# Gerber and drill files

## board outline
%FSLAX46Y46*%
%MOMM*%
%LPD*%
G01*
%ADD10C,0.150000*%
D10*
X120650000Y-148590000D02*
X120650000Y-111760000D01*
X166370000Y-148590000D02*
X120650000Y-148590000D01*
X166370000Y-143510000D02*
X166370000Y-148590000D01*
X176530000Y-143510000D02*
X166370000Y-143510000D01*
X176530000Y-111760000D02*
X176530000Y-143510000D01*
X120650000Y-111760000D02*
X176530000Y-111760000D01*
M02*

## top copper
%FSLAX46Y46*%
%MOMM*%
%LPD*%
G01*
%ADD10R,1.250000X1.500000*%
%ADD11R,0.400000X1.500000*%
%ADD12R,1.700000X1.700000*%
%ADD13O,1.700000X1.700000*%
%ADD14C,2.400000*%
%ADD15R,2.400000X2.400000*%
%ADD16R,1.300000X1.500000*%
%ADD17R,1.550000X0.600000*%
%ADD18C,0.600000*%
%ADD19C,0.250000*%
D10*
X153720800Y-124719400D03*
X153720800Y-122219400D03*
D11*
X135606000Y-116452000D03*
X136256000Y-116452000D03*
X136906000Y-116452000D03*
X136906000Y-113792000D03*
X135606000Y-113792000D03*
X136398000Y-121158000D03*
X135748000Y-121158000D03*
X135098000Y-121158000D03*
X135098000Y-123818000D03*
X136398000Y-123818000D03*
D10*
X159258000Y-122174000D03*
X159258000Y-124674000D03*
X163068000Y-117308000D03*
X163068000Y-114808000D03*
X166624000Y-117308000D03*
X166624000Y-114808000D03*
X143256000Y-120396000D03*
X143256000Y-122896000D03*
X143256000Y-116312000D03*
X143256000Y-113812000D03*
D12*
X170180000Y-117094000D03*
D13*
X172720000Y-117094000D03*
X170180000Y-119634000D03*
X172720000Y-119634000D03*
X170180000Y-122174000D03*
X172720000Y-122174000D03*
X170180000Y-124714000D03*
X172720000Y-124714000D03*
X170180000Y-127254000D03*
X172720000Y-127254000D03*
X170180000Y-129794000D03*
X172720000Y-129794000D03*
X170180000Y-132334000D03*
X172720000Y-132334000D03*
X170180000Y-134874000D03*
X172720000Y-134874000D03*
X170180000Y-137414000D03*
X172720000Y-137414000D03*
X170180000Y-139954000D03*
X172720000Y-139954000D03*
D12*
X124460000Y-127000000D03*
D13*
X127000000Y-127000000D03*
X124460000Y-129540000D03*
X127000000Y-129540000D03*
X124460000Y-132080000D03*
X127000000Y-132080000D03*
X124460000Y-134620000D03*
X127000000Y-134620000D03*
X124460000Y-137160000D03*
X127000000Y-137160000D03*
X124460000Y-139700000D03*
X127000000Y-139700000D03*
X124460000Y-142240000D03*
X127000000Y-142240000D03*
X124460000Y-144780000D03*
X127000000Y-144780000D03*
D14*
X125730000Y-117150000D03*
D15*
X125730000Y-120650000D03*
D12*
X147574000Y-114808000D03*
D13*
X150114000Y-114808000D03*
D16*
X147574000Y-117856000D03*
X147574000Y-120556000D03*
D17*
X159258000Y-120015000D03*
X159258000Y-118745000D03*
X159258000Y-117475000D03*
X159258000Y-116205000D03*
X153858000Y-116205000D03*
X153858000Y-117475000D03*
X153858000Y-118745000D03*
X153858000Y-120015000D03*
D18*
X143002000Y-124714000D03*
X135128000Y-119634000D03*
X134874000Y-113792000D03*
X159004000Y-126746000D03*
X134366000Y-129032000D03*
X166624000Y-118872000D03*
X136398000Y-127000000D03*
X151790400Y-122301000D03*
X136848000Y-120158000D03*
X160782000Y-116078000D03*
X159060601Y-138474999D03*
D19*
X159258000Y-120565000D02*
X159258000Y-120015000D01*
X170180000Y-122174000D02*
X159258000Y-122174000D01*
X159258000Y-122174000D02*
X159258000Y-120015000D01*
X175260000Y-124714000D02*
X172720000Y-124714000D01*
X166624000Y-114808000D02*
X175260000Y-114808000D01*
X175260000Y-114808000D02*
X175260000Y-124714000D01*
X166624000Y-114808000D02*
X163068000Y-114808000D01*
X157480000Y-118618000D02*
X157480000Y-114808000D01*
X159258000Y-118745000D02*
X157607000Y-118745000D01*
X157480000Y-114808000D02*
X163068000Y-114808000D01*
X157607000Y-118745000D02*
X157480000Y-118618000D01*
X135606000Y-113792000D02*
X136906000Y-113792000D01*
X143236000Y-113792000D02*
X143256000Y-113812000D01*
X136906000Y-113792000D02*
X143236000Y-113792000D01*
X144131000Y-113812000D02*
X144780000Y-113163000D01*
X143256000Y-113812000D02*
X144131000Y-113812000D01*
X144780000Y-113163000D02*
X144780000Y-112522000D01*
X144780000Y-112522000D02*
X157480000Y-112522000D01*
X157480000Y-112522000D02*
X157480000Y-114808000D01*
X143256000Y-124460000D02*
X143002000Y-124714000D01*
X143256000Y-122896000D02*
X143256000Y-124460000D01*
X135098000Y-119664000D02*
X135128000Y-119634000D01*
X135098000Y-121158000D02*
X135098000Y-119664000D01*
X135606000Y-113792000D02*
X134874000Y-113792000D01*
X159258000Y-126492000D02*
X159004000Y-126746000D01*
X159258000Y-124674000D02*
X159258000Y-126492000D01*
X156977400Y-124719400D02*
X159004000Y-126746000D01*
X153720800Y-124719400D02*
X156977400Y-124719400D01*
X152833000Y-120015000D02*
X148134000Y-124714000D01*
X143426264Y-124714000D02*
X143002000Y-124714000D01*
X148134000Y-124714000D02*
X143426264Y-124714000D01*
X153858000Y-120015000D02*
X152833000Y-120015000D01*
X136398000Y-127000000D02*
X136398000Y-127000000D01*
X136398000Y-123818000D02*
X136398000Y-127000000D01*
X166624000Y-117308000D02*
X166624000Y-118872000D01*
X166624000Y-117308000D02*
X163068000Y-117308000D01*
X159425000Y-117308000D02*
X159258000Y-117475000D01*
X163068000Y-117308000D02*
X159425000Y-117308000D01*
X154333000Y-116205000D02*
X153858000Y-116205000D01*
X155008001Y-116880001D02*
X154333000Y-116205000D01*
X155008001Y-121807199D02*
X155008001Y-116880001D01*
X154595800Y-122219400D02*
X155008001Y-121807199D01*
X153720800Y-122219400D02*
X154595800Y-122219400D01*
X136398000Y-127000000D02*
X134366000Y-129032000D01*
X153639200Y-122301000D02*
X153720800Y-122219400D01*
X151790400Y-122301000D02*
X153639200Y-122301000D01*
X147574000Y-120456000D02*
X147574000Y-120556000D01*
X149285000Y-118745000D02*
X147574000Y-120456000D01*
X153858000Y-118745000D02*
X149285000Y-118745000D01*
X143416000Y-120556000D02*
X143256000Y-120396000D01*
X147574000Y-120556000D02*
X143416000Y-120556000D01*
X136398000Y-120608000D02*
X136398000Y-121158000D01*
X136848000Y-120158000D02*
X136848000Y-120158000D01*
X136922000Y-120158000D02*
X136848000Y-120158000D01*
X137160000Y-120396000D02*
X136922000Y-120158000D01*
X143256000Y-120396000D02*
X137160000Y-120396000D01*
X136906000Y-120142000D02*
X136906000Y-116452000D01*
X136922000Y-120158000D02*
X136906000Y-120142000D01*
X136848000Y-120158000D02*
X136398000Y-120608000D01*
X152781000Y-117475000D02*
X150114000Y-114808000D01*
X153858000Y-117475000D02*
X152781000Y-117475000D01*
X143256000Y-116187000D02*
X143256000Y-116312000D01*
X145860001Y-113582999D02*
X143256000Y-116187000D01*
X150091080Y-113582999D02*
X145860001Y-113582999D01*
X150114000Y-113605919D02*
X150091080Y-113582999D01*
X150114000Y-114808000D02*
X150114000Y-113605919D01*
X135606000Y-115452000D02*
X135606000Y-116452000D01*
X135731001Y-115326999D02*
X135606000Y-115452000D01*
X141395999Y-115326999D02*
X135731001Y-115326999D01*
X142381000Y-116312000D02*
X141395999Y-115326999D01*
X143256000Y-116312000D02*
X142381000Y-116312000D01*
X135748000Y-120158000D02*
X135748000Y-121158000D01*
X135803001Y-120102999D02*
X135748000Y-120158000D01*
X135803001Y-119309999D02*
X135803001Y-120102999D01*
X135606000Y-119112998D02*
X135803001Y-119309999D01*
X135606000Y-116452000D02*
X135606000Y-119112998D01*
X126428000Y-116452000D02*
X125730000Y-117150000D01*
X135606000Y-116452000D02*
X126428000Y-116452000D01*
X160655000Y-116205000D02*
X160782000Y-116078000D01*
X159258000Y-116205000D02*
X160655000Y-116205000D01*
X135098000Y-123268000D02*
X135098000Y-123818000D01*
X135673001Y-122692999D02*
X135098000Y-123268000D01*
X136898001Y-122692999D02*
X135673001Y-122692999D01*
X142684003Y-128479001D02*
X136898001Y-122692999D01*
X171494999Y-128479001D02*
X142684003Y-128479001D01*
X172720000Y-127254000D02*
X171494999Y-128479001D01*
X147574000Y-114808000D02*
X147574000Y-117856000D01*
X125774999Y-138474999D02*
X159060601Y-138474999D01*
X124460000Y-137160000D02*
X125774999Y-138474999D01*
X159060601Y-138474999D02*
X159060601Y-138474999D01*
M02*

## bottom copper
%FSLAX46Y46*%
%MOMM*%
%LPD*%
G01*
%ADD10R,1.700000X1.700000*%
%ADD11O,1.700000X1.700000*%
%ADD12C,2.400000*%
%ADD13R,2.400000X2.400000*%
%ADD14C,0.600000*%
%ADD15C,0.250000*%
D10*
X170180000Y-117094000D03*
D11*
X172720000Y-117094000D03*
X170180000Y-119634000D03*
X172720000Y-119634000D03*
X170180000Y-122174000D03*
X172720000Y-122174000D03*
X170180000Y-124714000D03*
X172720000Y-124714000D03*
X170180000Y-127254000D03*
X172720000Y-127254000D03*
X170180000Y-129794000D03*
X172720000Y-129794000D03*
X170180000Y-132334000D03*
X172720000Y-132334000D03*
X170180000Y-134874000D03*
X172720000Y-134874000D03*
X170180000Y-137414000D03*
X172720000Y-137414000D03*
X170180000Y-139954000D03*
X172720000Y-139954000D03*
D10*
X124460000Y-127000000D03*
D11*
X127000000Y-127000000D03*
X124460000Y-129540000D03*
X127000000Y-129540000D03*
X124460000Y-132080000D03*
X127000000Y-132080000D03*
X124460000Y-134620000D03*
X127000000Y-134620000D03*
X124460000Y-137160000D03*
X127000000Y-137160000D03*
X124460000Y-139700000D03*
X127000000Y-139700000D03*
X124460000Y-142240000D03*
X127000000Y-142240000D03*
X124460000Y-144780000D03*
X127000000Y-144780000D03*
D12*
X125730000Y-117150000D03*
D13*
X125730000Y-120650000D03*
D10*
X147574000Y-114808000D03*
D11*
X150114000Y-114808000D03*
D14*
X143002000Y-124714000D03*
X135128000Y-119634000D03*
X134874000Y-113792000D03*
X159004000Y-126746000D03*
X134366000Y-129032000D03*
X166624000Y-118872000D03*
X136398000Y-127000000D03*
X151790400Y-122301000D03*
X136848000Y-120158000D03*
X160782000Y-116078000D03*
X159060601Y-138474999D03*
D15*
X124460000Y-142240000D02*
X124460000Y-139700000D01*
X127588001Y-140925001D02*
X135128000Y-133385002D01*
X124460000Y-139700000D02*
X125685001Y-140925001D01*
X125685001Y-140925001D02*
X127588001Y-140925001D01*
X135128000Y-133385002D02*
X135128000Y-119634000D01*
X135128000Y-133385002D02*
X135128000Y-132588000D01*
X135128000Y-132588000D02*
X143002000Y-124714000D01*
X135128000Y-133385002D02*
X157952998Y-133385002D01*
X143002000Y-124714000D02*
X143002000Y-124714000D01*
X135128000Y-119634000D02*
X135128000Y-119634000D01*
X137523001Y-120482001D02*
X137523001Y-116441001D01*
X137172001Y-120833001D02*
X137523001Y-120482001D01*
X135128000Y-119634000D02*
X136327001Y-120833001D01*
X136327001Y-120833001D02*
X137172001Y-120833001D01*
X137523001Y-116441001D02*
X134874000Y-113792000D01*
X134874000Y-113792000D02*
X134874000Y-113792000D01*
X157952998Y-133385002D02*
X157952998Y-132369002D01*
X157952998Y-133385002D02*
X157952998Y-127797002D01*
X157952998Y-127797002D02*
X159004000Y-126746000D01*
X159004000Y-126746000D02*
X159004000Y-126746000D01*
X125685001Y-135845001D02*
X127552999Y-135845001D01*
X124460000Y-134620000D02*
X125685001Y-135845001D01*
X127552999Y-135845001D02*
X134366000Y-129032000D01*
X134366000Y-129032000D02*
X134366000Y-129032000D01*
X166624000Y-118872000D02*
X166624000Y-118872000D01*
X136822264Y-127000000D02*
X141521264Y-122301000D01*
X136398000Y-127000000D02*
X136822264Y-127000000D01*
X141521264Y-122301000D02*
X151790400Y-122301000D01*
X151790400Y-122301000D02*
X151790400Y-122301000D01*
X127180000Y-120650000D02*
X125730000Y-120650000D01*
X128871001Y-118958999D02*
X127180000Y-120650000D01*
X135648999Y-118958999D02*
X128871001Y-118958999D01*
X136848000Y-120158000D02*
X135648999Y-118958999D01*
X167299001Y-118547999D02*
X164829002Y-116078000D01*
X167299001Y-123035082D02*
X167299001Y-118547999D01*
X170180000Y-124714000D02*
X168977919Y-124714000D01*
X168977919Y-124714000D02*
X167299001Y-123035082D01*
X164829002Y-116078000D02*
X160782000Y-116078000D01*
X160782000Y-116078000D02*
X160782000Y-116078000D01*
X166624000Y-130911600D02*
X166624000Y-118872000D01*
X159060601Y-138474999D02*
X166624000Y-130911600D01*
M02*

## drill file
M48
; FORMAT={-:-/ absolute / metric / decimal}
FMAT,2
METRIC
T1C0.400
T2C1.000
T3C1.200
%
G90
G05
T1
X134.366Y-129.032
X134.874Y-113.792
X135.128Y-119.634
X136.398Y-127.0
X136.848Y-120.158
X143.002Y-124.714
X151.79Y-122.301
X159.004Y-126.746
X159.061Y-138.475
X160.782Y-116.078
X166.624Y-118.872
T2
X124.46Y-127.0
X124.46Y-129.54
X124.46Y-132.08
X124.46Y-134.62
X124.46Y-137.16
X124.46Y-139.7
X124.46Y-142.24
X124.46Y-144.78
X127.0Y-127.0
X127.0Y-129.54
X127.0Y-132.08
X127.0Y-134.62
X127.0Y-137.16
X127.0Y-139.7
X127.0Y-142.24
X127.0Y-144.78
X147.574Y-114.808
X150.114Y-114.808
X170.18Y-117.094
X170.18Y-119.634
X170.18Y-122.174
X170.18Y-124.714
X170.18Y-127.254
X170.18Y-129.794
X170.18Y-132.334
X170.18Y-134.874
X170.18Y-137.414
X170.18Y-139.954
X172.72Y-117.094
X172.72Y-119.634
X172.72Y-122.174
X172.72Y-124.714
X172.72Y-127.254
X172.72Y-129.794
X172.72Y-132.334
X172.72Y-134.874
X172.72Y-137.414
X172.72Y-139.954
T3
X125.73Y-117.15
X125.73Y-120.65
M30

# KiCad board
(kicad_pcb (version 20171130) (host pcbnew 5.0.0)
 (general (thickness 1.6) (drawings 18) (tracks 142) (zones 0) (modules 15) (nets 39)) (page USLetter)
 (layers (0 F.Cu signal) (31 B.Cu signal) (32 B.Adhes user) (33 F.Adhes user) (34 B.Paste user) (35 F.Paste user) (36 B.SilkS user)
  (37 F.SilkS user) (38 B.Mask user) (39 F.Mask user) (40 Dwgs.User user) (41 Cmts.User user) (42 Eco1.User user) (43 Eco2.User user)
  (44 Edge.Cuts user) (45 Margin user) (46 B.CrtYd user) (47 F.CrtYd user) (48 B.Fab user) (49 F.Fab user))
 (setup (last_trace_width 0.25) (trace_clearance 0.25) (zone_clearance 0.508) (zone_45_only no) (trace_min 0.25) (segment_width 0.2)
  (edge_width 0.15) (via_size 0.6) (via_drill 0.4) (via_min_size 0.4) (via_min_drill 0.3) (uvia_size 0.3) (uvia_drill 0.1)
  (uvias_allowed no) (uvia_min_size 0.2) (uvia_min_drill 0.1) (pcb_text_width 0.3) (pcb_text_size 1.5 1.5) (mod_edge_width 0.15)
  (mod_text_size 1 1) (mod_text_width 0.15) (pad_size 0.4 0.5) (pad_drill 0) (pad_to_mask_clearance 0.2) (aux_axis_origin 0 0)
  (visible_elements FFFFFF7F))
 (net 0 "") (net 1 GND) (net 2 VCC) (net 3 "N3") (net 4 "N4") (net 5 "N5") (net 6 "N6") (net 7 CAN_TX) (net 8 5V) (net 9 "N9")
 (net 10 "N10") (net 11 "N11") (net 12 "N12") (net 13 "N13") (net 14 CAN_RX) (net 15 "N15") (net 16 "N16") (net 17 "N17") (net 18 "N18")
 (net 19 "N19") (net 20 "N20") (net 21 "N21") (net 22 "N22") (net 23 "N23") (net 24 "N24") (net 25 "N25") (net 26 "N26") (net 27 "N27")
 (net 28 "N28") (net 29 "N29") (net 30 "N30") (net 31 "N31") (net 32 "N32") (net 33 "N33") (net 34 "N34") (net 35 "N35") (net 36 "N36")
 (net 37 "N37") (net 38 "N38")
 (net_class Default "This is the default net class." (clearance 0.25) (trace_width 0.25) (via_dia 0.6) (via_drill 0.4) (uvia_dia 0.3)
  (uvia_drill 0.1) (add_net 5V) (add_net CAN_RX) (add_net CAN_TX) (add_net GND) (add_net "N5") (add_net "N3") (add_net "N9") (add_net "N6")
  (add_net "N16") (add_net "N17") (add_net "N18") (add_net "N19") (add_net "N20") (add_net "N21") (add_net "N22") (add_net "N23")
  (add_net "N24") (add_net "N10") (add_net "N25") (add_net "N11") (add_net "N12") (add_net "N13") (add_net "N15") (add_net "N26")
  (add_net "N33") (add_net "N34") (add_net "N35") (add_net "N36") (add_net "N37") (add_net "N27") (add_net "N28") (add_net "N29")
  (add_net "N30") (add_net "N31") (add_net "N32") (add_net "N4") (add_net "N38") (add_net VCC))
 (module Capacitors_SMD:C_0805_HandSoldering (layer F.Cu) (at 153.7208 123.4694 90)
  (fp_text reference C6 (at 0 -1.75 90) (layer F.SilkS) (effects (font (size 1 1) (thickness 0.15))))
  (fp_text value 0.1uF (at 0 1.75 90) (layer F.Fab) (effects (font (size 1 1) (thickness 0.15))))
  (pad 1 smd rect (at -1.25 0 90) (size 1.5 1.25) (layers F.Cu F.Paste F.Mask) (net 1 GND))
  (pad 2 smd rect (at 1.25 0 90) (size 1.5 1.25) (layers F.Cu F.Paste F.Mask) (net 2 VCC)))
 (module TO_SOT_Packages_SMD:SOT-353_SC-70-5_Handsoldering (layer F.Cu) (at 136.256 115.122 90)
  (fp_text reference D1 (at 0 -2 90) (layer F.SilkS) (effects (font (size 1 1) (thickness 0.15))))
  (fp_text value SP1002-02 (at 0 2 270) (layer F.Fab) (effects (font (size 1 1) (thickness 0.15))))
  (pad 1 smd rect (at -1.33 -0.65 90) (size 1.5 0.4) (layers F.Cu F.Paste F.Mask) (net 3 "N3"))
  (pad 2 smd rect (at -1.33 0 90) (size 1.5 0.4) (layers F.Cu F.Paste F.Mask) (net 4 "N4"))
  (pad 3 smd rect (at -1.33 0.65 90) (size 1.5 0.4) (layers F.Cu F.Paste F.Mask) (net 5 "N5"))
  (pad 4 smd rect (at 1.33 0.65 90) (size 1.5 0.4) (layers F.Cu F.Paste F.Mask) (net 1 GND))
  (pad 5 smd rect (at 1.33 -0.65 90) (size 1.5 0.4) (layers F.Cu F.Paste F.Mask) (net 1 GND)))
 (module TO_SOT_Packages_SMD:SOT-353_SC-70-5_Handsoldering (layer F.Cu) (at 135.748 122.488 270)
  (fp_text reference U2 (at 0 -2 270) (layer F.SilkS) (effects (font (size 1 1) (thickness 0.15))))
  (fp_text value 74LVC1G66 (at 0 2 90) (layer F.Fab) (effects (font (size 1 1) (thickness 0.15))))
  (pad 1 smd rect (at -1.33 -0.65 270) (size 1.5 0.4) (layers F.Cu F.Paste F.Mask) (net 5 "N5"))
  (pad 2 smd rect (at -1.33 0 270) (size 1.5 0.4) (layers F.Cu F.Paste F.Mask) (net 3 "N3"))
  (pad 3 smd rect (at -1.33 0.65 270) (size 1.5 0.4) (layers F.Cu F.Paste F.Mask) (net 1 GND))
  (pad 4 smd rect (at 1.33 0.65 270) (size 1.5 0.4) (layers F.Cu F.Paste F.Mask) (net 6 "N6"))
  (pad 5 smd rect (at 1.33 -0.65 270) (size 1.5 0.4) (layers F.Cu F.Paste F.Mask) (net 2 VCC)))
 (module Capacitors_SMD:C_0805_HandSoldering (layer F.Cu) (at 159.258 123.424 270)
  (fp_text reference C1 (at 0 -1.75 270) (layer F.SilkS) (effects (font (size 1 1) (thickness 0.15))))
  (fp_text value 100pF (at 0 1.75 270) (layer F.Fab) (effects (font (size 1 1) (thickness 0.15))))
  (pad 1 smd rect (at -1.25 0 270) (size 1.5 1.25) (layers F.Cu F.Paste F.Mask) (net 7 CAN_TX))
  (pad 2 smd rect (at 1.25 0 270) (size 1.5 1.25) (layers F.Cu F.Paste F.Mask) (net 1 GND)))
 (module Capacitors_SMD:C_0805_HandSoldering (layer F.Cu) (at 163.068 116.058 90)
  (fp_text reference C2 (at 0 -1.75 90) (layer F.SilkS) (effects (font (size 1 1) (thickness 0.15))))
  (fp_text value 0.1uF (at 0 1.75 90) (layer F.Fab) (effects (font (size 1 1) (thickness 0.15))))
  (pad 1 smd rect (at -1.25 0 90) (size 1.5 1.25) (layers F.Cu F.Paste F.Mask) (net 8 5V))
  (pad 2 smd rect (at 1.25 0 90) (size 1.5 1.25) (layers F.Cu F.Paste F.Mask) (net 1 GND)))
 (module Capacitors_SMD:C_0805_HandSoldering (layer F.Cu) (at 166.624 116.058 90)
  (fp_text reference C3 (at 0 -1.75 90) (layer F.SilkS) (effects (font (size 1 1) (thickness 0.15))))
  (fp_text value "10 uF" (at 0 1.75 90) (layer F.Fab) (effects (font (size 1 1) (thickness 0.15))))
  (pad 1 smd rect (at -1.25 0 90) (size 1.5 1.25) (layers F.Cu F.Paste F.Mask) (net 8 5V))
  (pad 2 smd rect (at 1.25 0 90) (size 1.5 1.25) (layers F.Cu F.Paste F.Mask) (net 1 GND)))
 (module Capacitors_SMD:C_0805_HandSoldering (layer F.Cu) (at 143.256 121.646 270)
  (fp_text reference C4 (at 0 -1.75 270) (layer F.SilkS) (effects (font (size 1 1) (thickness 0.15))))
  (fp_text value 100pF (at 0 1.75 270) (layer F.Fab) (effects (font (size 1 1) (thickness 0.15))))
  (pad 1 smd rect (at -1.25 0 270) (size 1.5 1.25) (layers F.Cu F.Paste F.Mask) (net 5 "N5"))
  (pad 2 smd rect (at 1.25 0 270) (size 1.5 1.25) (layers F.Cu F.Paste F.Mask) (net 1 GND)))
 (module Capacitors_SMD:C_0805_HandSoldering (layer F.Cu) (at 143.256 115.062 90)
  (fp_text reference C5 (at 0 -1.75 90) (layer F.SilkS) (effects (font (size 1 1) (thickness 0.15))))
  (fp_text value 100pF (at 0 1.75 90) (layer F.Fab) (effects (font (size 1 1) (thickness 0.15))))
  (pad 1 smd rect (at -1.25 0 90) (size 1.5 1.25) (layers F.Cu F.Paste F.Mask) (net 3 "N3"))
  (pad 2 smd rect (at 1.25 0 90) (size 1.5 1.25) (layers F.Cu F.Paste F.Mask) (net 1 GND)))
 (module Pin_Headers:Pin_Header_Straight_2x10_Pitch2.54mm (layer F.Cu) (at 170.18 117.094)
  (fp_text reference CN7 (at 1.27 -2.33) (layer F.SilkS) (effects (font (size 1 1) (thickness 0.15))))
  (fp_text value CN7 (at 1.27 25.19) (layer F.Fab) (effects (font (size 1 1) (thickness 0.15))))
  (pad 1 thru_hole rect (at 0 0) (size 1.7 1.7) (drill 1) (layers *.Cu *.Mask) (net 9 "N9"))
  (pad 2 thru_hole oval (at 2.54 0) (size 1.7 1.7) (drill 1) (layers *.Cu *.Mask) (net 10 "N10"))
  (pad 3 thru_hole oval (at 0 2.54) (size 1.7 1.7) (drill 1) (layers *.Cu *.Mask) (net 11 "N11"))
  (pad 4 thru_hole oval (at 2.54 2.54) (size 1.7 1.7) (drill 1) (layers *.Cu *.Mask) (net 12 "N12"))
  (pad 5 thru_hole oval (at 0 5.08) (size 1.7 1.7) (drill 1) (layers *.Cu *.Mask) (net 7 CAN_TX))
  (pad 6 thru_hole oval (at 2.54 5.08) (size 1.7 1.7) (drill 1) (layers *.Cu *.Mask) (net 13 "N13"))
  (pad 7 thru_hole oval (at 0 7.62) (size 1.7 1.7) (drill 1) (layers *.Cu *.Mask) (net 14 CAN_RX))
  (pad 8 thru_hole oval (at 2.54 7.62) (size 1.7 1.7) (drill 1) (layers *.Cu *.Mask) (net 1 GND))
  (pad 9 thru_hole oval (at 0 10.16) (size 1.7 1.7) (drill 1) (layers *.Cu *.Mask) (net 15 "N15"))
  (pad 10 thru_hole oval (at 2.54 10.16) (size 1.7 1.7) (drill 1) (layers *.Cu *.Mask) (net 6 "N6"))
  (pad 11 thru_hole oval (at 0 12.7) (size 1.7 1.7) (drill 1) (layers *.Cu *.Mask) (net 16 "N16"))
  (pad 12 thru_hole oval (at 2.54 12.7) (size 1.7 1.7) (drill 1) (layers *.Cu *.Mask) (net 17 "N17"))
  (pad 13 thru_hole oval (at 0 15.24) (size 1.7 1.7) (drill 1) (layers *.Cu *.Mask) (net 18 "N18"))
  (pad 14 thru_hole oval (at 2.54 15.24) (size 1.7 1.7) (drill 1) (layers *.Cu *.Mask) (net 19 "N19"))
  (pad 15 thru_hole oval (at 0 17.78) (size 1.7 1.7) (drill 1) (layers *.Cu *.Mask) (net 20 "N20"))
  (pad 16 thru_hole oval (at 2.54 17.78) (size 1.7 1.7) (drill 1) (layers *.Cu *.Mask) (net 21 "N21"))
  (pad 17 thru_hole oval (at 0 20.32) (size 1.7 1.7) (drill 1) (layers *.Cu *.Mask) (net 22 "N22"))
  (pad 18 thru_hole oval (at 2.54 20.32) (size 1.7 1.7) (drill 1) (layers *.Cu *.Mask) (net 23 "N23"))
  (pad 19 thru_hole oval (at 0 22.86) (size 1.7 1.7) (drill 1) (layers *.Cu *.Mask) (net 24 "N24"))
  (pad 20 thru_hole oval (at 2.54 22.86) (size 1.7 1.7) (drill 1) (layers *.Cu *.Mask) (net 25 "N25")))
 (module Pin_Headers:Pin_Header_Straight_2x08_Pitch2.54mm (layer F.Cu) (at 124.46 127)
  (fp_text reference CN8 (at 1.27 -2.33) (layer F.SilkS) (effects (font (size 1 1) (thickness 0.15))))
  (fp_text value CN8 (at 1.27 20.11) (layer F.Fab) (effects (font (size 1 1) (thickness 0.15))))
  (pad 1 thru_hole rect (at 0 0) (size 1.7 1.7) (drill 1) (layers *.Cu *.Mask) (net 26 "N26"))
  (pad 2 thru_hole oval (at 2.54 0) (size 1.7 1.7) (drill 1) (layers *.Cu *.Mask) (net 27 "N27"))
  (pad 3 thru_hole oval (at 0 2.54) (size 1.7 1.7) (drill 1) (layers *.Cu *.Mask) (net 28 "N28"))
  (pad 4 thru_hole oval (at 2.54 2.54) (size 1.7 1.7) (drill 1) (layers *.Cu *.Mask) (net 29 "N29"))
  (pad 5 thru_hole oval (at 0 5.08) (size 1.7 1.7) (drill 1) (layers *.Cu *.Mask) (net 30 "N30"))
  (pad 6 thru_hole oval (at 2.54 5.08) (size 1.7 1.7) (drill 1) (layers *.Cu *.Mask) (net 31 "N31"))
  (pad 7 thru_hole oval (at 0 7.62) (size 1.7 1.7) (drill 1) (layers *.Cu *.Mask) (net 2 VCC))
  (pad 8 thru_hole oval (at 2.54 7.62) (size 1.7 1.7) (drill 1) (layers *.Cu *.Mask) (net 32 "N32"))
  (pad 9 thru_hole oval (at 0 10.16) (size 1.7 1.7) (drill 1) (layers *.Cu *.Mask) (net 8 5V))
  (pad 10 thru_hole oval (at 2.54 10.16) (size 1.7 1.7) (drill 1) (layers *.Cu *.Mask) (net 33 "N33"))
  (pad 11 thru_hole oval (at 0 12.7) (size 1.7 1.7) (drill 1) (layers *.Cu *.Mask) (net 1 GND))
  (pad 12 thru_hole oval (at 2.54 12.7) (size 1.7 1.7) (drill 1) (layers *.Cu *.Mask) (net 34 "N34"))
  (pad 13 thru_hole oval (at 0 15.24) (size 1.7 1.7) (drill 1) (layers *.Cu *.Mask) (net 1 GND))
  (pad 14 thru_hole oval (at 2.54 15.24) (size 1.7 1.7) (drill 1) (layers *.Cu *.Mask) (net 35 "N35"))
  (pad 15 thru_hole oval (at 0 17.78) (size 1.7 1.7) (drill 1) (layers *.Cu *.Mask) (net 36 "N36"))
  (pad 16 thru_hole oval (at 2.54 17.78) (size 1.7 1.7) (drill 1) (layers *.Cu *.Mask) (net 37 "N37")))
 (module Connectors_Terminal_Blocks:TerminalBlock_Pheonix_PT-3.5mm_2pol (layer F.Cu) (at 125.73 120.65 90)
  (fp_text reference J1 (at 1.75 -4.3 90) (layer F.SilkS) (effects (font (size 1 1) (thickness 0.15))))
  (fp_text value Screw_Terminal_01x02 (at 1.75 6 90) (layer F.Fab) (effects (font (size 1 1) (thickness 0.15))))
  (pad 2 thru_hole circle (at 3.5 0 90) (size 2.4 2.4) (drill 1.2) (layers *.Cu *.Mask) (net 3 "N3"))
  (pad 1 thru_hole rect (at 0 0 90) (size 2.4 2.4) (drill 1.2) (layers *.Cu *.Mask) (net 5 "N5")))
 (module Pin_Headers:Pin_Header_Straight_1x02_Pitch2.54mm (layer F.Cu) (at 147.574 114.808 90)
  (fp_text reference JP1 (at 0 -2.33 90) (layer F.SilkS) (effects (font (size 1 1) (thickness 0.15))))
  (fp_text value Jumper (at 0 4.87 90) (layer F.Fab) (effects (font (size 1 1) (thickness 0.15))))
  (pad 1 thru_hole rect (at 0 0 90) (size 1.7 1.7) (drill 1) (layers *.Cu *.Mask) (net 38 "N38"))
  (pad 2 thru_hole oval (at 0 2.54 90) (size 1.7 1.7) (drill 1) (layers *.Cu *.Mask) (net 3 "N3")))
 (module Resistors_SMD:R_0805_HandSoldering (layer F.Cu) (at 147.574 119.206 270)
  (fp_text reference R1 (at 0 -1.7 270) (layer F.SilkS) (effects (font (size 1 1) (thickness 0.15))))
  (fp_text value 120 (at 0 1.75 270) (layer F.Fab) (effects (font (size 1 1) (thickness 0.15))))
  (pad 1 smd rect (at -1.35 0 270) (size 1.5 1.3) (layers F.Cu F.Paste F.Mask) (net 38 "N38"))
  (pad 2 smd rect (at 1.35 0 270) (size 1.5 1.3) (layers F.Cu F.Paste F.Mask) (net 5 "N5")))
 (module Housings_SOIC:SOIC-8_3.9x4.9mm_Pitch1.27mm (layer F.Cu) (at 156.558 118.11 180)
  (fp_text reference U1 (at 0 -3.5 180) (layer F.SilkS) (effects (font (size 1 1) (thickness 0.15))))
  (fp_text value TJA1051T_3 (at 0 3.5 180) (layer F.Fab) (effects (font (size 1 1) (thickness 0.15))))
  (pad 1 smd rect (at -2.7 -1.905 180) (size 1.55 0.6) (layers F.Cu F.Paste F.Mask) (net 7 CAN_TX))
  (pad 2 smd rect (at -2.7 -0.635 180) (size 1.55 0.6) (layers F.Cu F.Paste F.Mask) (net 1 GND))
  (pad 3 smd rect (at -2.7 0.635 180) (size 1.55 0.6) (layers F.Cu F.Paste F.Mask) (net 8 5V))
  (pad 4 smd rect (at -2.7 1.905 180) (size 1.55 0.6) (layers F.Cu F.Paste F.Mask) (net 14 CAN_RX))
  (pad 5 smd rect (at 2.7 1.905 180) (size 1.55 0.6) (layers F.Cu F.Paste F.Mask) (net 2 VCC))
  (pad 6 smd rect (at 2.7 0.635 180) (size 1.55 0.6) (layers F.Cu F.Paste F.Mask) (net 3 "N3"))
  (pad 7 smd rect (at 2.7 -0.635 180) (size 1.55 0.6) (layers F.Cu F.Paste F.Mask) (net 5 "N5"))
  (pad 8 smd rect (at 2.7 -1.905 180) (size 1.55 0.6) (layers F.Cu F.Paste F.Mask) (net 1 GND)))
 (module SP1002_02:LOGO (layer B.Cu) (at 147.32 134.2898)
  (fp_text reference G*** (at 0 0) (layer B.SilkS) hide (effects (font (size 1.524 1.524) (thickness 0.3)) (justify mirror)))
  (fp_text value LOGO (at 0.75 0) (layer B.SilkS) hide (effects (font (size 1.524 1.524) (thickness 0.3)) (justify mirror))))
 (gr_line (start 120.65 148.59) (end 120.65 111.76) (angle 90) (layer Edge.Cuts) (width 0.15))
 (gr_line (start 166.37 148.59) (end 120.65 148.59) (angle 90) (layer Edge.Cuts) (width 0.15))
 (gr_line (start 166.37 143.51) (end 166.37 148.59) (angle 90) (layer Edge.Cuts) (width 0.15))
 (gr_line (start 176.53 143.51) (end 166.37 143.51) (angle 90) (layer Edge.Cuts) (width 0.15))
 (gr_line (start 176.53 111.76) (end 176.53 143.51) (angle 90) (layer Edge.Cuts) (width 0.15))
 (gr_line (start 120.65 111.76) (end 176.53 111.76) (angle 90) (layer Edge.Cuts) (width 0.15))
 (segment (start 159.258 120.565) (end 159.258 120.015) (width 0.25) (layer F.Cu) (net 7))
 (segment (start 170.18 122.174) (end 159.258 122.174) (width 0.25) (layer F.Cu) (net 7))
 (segment (start 159.258 122.174) (end 159.258 120.015) (width 0.25) (layer F.Cu) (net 7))
 (segment (start 124.46 142.24) (end 124.46 139.7) (width 0.25) (layer B.Cu) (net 1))
 (segment (start 175.26 124.714) (end 172.72 124.714) (width 0.25) (layer F.Cu) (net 1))
 (segment (start 166.624 114.808) (end 175.26 114.808) (width 0.25) (layer F.Cu) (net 1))
 (segment (start 175.26 114.808) (end 175.26 124.714) (width 0.25) (layer F.Cu) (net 1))
 (segment (start 166.624 114.808) (end 163.068 114.808) (width 0.25) (layer F.Cu) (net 1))
 (segment (start 157.48 118.618) (end 157.48 114.808) (width 0.25) (layer F.Cu) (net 1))
 (segment (start 159.258 118.745) (end 157.607 118.745) (width 0.25) (layer F.Cu) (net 1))
 (segment (start 157.48 114.808) (end 163.068 114.808) (width 0.25) (layer F.Cu) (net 1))
 (segment (start 157.607 118.745) (end 157.48 118.618) (width 0.25) (layer F.Cu) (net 1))
 (segment (start 135.606 113.792) (end 136.906 113.792) (width 0.25) (layer F.Cu) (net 1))
 (segment (start 143.236 113.792) (end 143.256 113.812) (width 0.25) (layer F.Cu) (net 1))
 (segment (start 136.906 113.792) (end 143.236 113.792) (width 0.25) (layer F.Cu) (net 1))
 (segment (start 144.131 113.812) (end 144.78 113.163) (width 0.25) (layer F.Cu) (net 1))
 (segment (start 143.256 113.812) (end 144.131 113.812) (width 0.25) (layer F.Cu) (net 1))
 (segment (start 144.78 113.163) (end 144.78 112.522) (width 0.25) (layer F.Cu) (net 1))
 (segment (start 144.78 112.522) (end 157.48 112.522) (width 0.25) (layer F.Cu) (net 1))
 (segment (start 157.48 112.522) (end 157.48 114.808) (width 0.25) (layer F.Cu) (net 1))
 (segment (start 127.588001 140.925001) (end 135.128 133.385002) (width 0.25) (layer B.Cu) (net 1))
 (segment (start 124.46 139.7) (end 125.685001 140.925001) (width 0.25) (layer B.Cu) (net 1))
 (segment (start 125.685001 140.925001) (end 127.588001 140.925001) (width 0.25) (layer B.Cu) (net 1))
 (segment (start 135.128 133.385002) (end 135.128 119.634) (width 0.25) (layer B.Cu) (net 1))
 (segment (start 135.128 133.385002) (end 135.128 132.588) (width 0.25) (layer B.Cu) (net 1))
 (segment (start 135.128 132.588) (end 143.002 124.714) (width 0.25) (layer B.Cu) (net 1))
 (segment (start 135.128 133.385002) (end 157.952998 133.385002) (width 0.25) (layer B.Cu) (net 1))
 (segment (start 143.002 124.714) (end 143.002 124.714) (width 0.25) (layer B.Cu) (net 1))
 (via (at 143.002 124.714) (size 0.6) (drill 0.4) (layers F.Cu B.Cu) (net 1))
 (segment (start 135.128 119.634) (end 135.128 119.634) (width 0.25) (layer B.Cu) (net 1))
 (via (at 135.128 119.634) (size 0.6) (drill 0.4) (layers F.Cu B.Cu) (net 1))
 (segment (start 143.256 124.46) (end 143.002 124.714) (width 0.25) (layer F.Cu) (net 1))
 (segment (start 143.256 122.896) (end 143.256 124.46) (width 0.25) (layer F.Cu) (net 1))
 (segment (start 135.098 119.664) (end 135.128 119.634) (width 0.25) (layer F.Cu) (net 1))
 (segment (start 135.098 121.158) (end 135.098 119.664) (width 0.25) (layer F.Cu) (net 1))
 (segment (start 137.523001 120.482001) (end 137.523001 116.441001) (width 0.25) (layer B.Cu) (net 1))
 (segment (start 137.172001 120.833001) (end 137.523001 120.482001) (width 0.25) (layer B.Cu) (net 1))
 (segment (start 135.128 119.634) (end 136.327001 120.833001) (width 0.25) (layer B.Cu) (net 1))
 (segment (start 136.327001 120.833001) (end 137.172001 120.833001) (width 0.25) (layer B.Cu) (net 1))
 (segment (start 137.523001 116.441001) (end 134.874 113.792) (width 0.25) (layer B.Cu) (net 1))
 (segment (start 134.874 113.792) (end 134.874 113.792) (width 0.25) (layer B.Cu) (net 1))
 (via (at 134.874 113.792) (size 0.6) (drill 0.4) (layers F.Cu B.Cu) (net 1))
 (segment (start 135.606 113.792) (end 134.874 113.792) (width 0.25) (layer F.Cu) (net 1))
 (segment (start 157.952998 133.385002) (end 157.952998 132.369002) (width 0.25) (layer B.Cu) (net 1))
 (segment (start 157.952998 133.385002) (end 157.952998 127.797002) (width 0.25) (layer B.Cu) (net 1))
 (segment (start 157.952998 127.797002) (end 159.004 126.746) (width 0.25) (layer B.Cu) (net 1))
 (segment (start 159.004 126.746) (end 159.004 126.746) (width 0.25) (layer B.Cu) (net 1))
 (via (at 159.004 126.746) (size 0.6) (drill 0.4) (layers F.Cu B.Cu) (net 1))
 (segment (start 159.258 126.492) (end 159.004 126.746) (width 0.25) (layer F.Cu) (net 1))
 (segment (start 159.258 124.674) (end 159.258 126.492) (width 0.25) (layer F.Cu) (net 1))
 (segment (start 156.9774 124.7194) (end 159.004 126.746) (width 0.25) (layer F.Cu) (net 1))
 (segment (start 153.7208 124.7194) (end 156.9774 124.7194) (width 0.25) (layer F.Cu) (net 1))
 (segment (start 152.833 120.015) (end 148.134 124.714) (width 0.25) (layer F.Cu) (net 1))
 (segment (start 143.426264 124.714) (end 143.002 124.714) (width 0.25) (layer F.Cu) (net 1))
 (segment (start 148.134 124.714) (end 143.426264 124.714) (width 0.25) (layer F.Cu) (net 1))
 (segment (start 153.858 120.015) (end 152.833 120.015) (width 0.25) (layer F.Cu) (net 1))
 (segment (start 125.685001 135.845001) (end 127.552999 135.845001) (width 0.25) (layer B.Cu) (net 2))
 (segment (start 124.46 134.62) (end 125.685001 135.845001) (width 0.25) (layer B.Cu) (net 2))
 (segment (start 127.552999 135.845001) (end 134.366 129.032) (width 0.25) (layer B.Cu) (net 2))
 (segment (start 134.366 129.032) (end 134.366 129.032) (width 0.25) (layer B.Cu) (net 2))
 (via (at 134.366 129.032) (size 0.6) (drill 0.4) (layers F.Cu B.Cu) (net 2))
 (segment (start 136.398 127) (end 136.398 127) (width 0.25) (layer F.Cu) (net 2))
 (segment (start 136.398 123.818) (end 136.398 127) (width 0.25) (layer F.Cu) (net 2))
 (segment (start 166.624 118.872) (end 166.624 118.872) (width 0.25) (layer B.Cu) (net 8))
 (via (at 166.624 118.872) (size 0.6) (drill 0.4) (layers F.Cu B.Cu) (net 8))
 (segment (start 166.624 117.308) (end 166.624 118.872) (width 0.25) (layer F.Cu) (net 8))
 (segment (start 166.624 117.308) (end 163.068 117.308) (width 0.25) (layer F.Cu) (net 8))
 (segment (start 159.425 117.308) (end 159.258 117.475) (width 0.25) (layer F.Cu) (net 8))
 (segment (start 163.068 117.308) (end 159.425 117.308) (width 0.25) (layer F.Cu) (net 8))
 (segment (start 154.333 116.205) (end 153.858 116.205) (width 0.25) (layer F.Cu) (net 2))
 (segment (start 155.008001 116.880001) (end 154.333 116.205) (width 0.25) (layer F.Cu) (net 2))
 (segment (start 155.008001 121.807199) (end 155.008001 116.880001) (width 0.25) (layer F.Cu) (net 2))
 (segment (start 154.5958 122.2194) (end 155.008001 121.807199) (width 0.25) (layer F.Cu) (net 2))
 (segment (start 153.7208 122.2194) (end 154.5958 122.2194) (width 0.25) (layer F.Cu) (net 2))
 (segment (start 136.398 127) (end 134.366 129.032) (width 0.25) (layer F.Cu) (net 2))
 (via (at 136.398 127) (size 0.6) (drill 0.4) (layers F.Cu B.Cu) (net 2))
 (segment (start 136.822264 127) (end 141.521264 122.301) (width 0.25) (layer B.Cu) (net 2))
 (segment (start 136.398 127) (end 136.822264 127) (width 0.25) (layer B.Cu) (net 2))
 (segment (start 141.521264 122.301) (end 151.7904 122.301) (width 0.25) (layer B.Cu) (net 2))
 (segment (start 151.7904 122.301) (end 151.7904 122.301) (width 0.25) (layer B.Cu) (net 2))
 (via (at 151.7904 122.301) (size 0.6) (drill 0.4) (layers F.Cu B.Cu) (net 2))
 (segment (start 153.6392 122.301) (end 153.7208 122.2194) (width 0.25) (layer F.Cu) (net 2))
 (segment (start 151.7904 122.301) (end 153.6392 122.301) (width 0.25) (layer F.Cu) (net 2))
 (segment (start 147.574 120.456) (end 147.574 120.556) (width 0.25) (layer F.Cu) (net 5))
 (segment (start 149.285 118.745) (end 147.574 120.456) (width 0.25) (layer F.Cu) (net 5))
 (segment (start 153.858 118.745) (end 149.285 118.745) (width 0.25) (layer F.Cu) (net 5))
 (segment (start 143.416 120.556) (end 143.256 120.396) (width 0.25) (layer F.Cu) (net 5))
 (segment (start 147.574 120.556) (end 143.416 120.556) (width 0.25) (layer F.Cu) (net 5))
 (segment (start 136.398 120.608) (end 136.398 121.158) (width 0.25) (layer F.Cu) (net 5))
 (segment (start 136.848 120.158) (end 136.848 120.158) (width 0.25) (layer F.Cu) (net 5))
 (segment (start 136.922 120.158) (end 136.848 120.158) (width 0.25) (layer F.Cu) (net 5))
 (segment (start 137.16 120.396) (end 136.922 120.158) (width 0.25) (layer F.Cu) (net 5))
 (segment (start 143.256 120.396) (end 137.16 120.396) (width 0.25) (layer F.Cu) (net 5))
 (segment (start 136.906 120.142) (end 136.906 116.452) (width 0.25) (layer F.Cu) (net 5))
 (segment (start 136.922 120.158) (end 136.906 120.142) (width 0.25) (layer F.Cu) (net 5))
 (segment (start 136.848 120.158) (end 136.398 120.608) (width 0.25) (layer F.Cu) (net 5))
 (via (at 136.848 120.158) (size 0.6) (drill 0.4) (layers F.Cu B.Cu) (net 5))
 (segment (start 127.18 120.65) (end 125.73 120.65) (width 0.25) (layer B.Cu) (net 5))
 (segment (start 128.871001 118.958999) (end 127.18 120.65) (width 0.25) (layer B.Cu) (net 5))
 (segment (start 135.648999 118.958999) (end 128.871001 118.958999) (width 0.25) (layer B.Cu) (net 5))
 (segment (start 136.848 120.158) (end 135.648999 118.958999) (width 0.25) (layer B.Cu) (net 5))
 (segment (start 152.781 117.475) (end 150.114 114.808) (width 0.25) (layer F.Cu) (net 3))
 (segment (start 153.858 117.475) (end 152.781 117.475) (width 0.25) (layer F.Cu) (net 3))
 (segment (start 143.256 116.187) (end 143.256 116.312) (width 0.25) (layer F.Cu) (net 3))
 (segment (start 145.860001 113.582999) (end 143.256 116.187) (width 0.25) (layer F.Cu) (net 3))
 (segment (start 150.09108 113.582999) (end 145.860001 113.582999) (width 0.25) (layer F.Cu) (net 3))
 (segment (start 150.114 113.605919) (end 150.09108 113.582999) (width 0.25) (layer F.Cu) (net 3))
 (segment (start 150.114 114.808) (end 150.114 113.605919) (width 0.25) (layer F.Cu) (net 3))
 (segment (start 135.606 115.452) (end 135.606 116.452) (width 0.25) (layer F.Cu) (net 3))
 (segment (start 135.731001 115.326999) (end 135.606 115.452) (width 0.25) (layer F.Cu) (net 3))
 (segment (start 141.395999 115.326999) (end 135.731001 115.326999) (width 0.25) (layer F.Cu) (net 3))
 (segment (start 142.381 116.312) (end 141.395999 115.326999) (width 0.25) (layer F.Cu) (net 3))
 (segment (start 143.256 116.312) (end 142.381 116.312) (width 0.25) (layer F.Cu) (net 3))
 (segment (start 135.748 120.158) (end 135.748 121.158) (width 0.25) (layer F.Cu) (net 3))
 (segment (start 135.803001 120.102999) (end 135.748 120.158) (width 0.25) (layer F.Cu) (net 3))
 (segment (start 135.803001 119.309999) (end 135.803001 120.102999) (width 0.25) (layer F.Cu) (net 3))
 (segment (start 135.606 119.112998) (end 135.803001 119.309999) (width 0.25) (layer F.Cu) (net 3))
 (segment (start 135.606 116.452) (end 135.606 119.112998) (width 0.25) (layer F.Cu) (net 3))
 (segment (start 126.428 116.452) (end 125.73 117.15) (width 0.25) (layer F.Cu) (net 3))
 (segment (start 135.606 116.452) (end 126.428 116.452) (width 0.25) (layer F.Cu) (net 3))
 (segment (start 167.299001 118.547999) (end 164.829002 116.078) (width 0.25) (layer B.Cu) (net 14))
 (segment (start 167.299001 123.035082) (end 167.299001 118.547999) (width 0.25) (layer B.Cu) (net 14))
 (segment (start 170.18 124.714) (end 168.977919 124.714) (width 0.25) (layer B.Cu) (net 14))
 (segment (start 168.977919 124.714) (end 167.299001 123.035082) (width 0.25) (layer B.Cu) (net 14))
 (segment (start 164.829002 116.078) (end 160.782 116.078) (width 0.25) (layer B.Cu) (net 14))
 (segment (start 160.782 116.078) (end 160.782 116.078) (width 0.25) (layer B.Cu) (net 14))
 (via (at 160.782 116.078) (size 0.6) (drill 0.4) (layers F.Cu B.Cu) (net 14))
 (segment (start 160.655 116.205) (end 160.782 116.078) (width 0.25) (layer F.Cu) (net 14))
 (segment (start 159.258 116.205) (end 160.655 116.205) (width 0.25) (layer F.Cu) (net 14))
 (segment (start 135.098 123.268) (end 135.098 123.818) (width 0.25) (layer F.Cu) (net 6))
 (segment (start 135.673001 122.692999) (end 135.098 123.268) (width 0.25) (layer F.Cu) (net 6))
 (segment (start 136.898001 122.692999) (end 135.673001 122.692999) (width 0.25) (layer F.Cu) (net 6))
 (segment (start 142.684003 128.479001) (end 136.898001 122.692999) (width 0.25) (layer F.Cu) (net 6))
 (segment (start 171.494999 128.479001) (end 142.684003 128.479001) (width 0.25) (layer F.Cu) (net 6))
 (segment (start 172.72 127.254) (end 171.494999 128.479001) (width 0.25) (layer F.Cu) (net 6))
 (segment (start 147.574 114.808) (end 147.574 117.856) (width 0.25) (layer F.Cu) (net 38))
 (segment (start 125.774999 138.474999) (end 159.060601 138.474999) (width 0.25) (layer F.Cu) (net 8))
 (segment (start 124.46 137.16) (end 125.774999 138.474999) (width 0.25) (layer F.Cu) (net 8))
 (segment (start 159.060601 138.474999) (end 159.060601 138.474999) (width 0.25) (layer F.Cu) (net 8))
 (via (at 159.060601 138.474999) (size 0.6) (drill 0.4) (layers F.Cu B.Cu) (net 8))
 (segment (start 166.624 130.9116) (end 166.624 118.872) (width 0.25) (layer B.Cu) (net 8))
 (segment (start 159.060601 138.474999) (end 166.624 130.9116) (width 0.25) (layer B.Cu) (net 8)))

